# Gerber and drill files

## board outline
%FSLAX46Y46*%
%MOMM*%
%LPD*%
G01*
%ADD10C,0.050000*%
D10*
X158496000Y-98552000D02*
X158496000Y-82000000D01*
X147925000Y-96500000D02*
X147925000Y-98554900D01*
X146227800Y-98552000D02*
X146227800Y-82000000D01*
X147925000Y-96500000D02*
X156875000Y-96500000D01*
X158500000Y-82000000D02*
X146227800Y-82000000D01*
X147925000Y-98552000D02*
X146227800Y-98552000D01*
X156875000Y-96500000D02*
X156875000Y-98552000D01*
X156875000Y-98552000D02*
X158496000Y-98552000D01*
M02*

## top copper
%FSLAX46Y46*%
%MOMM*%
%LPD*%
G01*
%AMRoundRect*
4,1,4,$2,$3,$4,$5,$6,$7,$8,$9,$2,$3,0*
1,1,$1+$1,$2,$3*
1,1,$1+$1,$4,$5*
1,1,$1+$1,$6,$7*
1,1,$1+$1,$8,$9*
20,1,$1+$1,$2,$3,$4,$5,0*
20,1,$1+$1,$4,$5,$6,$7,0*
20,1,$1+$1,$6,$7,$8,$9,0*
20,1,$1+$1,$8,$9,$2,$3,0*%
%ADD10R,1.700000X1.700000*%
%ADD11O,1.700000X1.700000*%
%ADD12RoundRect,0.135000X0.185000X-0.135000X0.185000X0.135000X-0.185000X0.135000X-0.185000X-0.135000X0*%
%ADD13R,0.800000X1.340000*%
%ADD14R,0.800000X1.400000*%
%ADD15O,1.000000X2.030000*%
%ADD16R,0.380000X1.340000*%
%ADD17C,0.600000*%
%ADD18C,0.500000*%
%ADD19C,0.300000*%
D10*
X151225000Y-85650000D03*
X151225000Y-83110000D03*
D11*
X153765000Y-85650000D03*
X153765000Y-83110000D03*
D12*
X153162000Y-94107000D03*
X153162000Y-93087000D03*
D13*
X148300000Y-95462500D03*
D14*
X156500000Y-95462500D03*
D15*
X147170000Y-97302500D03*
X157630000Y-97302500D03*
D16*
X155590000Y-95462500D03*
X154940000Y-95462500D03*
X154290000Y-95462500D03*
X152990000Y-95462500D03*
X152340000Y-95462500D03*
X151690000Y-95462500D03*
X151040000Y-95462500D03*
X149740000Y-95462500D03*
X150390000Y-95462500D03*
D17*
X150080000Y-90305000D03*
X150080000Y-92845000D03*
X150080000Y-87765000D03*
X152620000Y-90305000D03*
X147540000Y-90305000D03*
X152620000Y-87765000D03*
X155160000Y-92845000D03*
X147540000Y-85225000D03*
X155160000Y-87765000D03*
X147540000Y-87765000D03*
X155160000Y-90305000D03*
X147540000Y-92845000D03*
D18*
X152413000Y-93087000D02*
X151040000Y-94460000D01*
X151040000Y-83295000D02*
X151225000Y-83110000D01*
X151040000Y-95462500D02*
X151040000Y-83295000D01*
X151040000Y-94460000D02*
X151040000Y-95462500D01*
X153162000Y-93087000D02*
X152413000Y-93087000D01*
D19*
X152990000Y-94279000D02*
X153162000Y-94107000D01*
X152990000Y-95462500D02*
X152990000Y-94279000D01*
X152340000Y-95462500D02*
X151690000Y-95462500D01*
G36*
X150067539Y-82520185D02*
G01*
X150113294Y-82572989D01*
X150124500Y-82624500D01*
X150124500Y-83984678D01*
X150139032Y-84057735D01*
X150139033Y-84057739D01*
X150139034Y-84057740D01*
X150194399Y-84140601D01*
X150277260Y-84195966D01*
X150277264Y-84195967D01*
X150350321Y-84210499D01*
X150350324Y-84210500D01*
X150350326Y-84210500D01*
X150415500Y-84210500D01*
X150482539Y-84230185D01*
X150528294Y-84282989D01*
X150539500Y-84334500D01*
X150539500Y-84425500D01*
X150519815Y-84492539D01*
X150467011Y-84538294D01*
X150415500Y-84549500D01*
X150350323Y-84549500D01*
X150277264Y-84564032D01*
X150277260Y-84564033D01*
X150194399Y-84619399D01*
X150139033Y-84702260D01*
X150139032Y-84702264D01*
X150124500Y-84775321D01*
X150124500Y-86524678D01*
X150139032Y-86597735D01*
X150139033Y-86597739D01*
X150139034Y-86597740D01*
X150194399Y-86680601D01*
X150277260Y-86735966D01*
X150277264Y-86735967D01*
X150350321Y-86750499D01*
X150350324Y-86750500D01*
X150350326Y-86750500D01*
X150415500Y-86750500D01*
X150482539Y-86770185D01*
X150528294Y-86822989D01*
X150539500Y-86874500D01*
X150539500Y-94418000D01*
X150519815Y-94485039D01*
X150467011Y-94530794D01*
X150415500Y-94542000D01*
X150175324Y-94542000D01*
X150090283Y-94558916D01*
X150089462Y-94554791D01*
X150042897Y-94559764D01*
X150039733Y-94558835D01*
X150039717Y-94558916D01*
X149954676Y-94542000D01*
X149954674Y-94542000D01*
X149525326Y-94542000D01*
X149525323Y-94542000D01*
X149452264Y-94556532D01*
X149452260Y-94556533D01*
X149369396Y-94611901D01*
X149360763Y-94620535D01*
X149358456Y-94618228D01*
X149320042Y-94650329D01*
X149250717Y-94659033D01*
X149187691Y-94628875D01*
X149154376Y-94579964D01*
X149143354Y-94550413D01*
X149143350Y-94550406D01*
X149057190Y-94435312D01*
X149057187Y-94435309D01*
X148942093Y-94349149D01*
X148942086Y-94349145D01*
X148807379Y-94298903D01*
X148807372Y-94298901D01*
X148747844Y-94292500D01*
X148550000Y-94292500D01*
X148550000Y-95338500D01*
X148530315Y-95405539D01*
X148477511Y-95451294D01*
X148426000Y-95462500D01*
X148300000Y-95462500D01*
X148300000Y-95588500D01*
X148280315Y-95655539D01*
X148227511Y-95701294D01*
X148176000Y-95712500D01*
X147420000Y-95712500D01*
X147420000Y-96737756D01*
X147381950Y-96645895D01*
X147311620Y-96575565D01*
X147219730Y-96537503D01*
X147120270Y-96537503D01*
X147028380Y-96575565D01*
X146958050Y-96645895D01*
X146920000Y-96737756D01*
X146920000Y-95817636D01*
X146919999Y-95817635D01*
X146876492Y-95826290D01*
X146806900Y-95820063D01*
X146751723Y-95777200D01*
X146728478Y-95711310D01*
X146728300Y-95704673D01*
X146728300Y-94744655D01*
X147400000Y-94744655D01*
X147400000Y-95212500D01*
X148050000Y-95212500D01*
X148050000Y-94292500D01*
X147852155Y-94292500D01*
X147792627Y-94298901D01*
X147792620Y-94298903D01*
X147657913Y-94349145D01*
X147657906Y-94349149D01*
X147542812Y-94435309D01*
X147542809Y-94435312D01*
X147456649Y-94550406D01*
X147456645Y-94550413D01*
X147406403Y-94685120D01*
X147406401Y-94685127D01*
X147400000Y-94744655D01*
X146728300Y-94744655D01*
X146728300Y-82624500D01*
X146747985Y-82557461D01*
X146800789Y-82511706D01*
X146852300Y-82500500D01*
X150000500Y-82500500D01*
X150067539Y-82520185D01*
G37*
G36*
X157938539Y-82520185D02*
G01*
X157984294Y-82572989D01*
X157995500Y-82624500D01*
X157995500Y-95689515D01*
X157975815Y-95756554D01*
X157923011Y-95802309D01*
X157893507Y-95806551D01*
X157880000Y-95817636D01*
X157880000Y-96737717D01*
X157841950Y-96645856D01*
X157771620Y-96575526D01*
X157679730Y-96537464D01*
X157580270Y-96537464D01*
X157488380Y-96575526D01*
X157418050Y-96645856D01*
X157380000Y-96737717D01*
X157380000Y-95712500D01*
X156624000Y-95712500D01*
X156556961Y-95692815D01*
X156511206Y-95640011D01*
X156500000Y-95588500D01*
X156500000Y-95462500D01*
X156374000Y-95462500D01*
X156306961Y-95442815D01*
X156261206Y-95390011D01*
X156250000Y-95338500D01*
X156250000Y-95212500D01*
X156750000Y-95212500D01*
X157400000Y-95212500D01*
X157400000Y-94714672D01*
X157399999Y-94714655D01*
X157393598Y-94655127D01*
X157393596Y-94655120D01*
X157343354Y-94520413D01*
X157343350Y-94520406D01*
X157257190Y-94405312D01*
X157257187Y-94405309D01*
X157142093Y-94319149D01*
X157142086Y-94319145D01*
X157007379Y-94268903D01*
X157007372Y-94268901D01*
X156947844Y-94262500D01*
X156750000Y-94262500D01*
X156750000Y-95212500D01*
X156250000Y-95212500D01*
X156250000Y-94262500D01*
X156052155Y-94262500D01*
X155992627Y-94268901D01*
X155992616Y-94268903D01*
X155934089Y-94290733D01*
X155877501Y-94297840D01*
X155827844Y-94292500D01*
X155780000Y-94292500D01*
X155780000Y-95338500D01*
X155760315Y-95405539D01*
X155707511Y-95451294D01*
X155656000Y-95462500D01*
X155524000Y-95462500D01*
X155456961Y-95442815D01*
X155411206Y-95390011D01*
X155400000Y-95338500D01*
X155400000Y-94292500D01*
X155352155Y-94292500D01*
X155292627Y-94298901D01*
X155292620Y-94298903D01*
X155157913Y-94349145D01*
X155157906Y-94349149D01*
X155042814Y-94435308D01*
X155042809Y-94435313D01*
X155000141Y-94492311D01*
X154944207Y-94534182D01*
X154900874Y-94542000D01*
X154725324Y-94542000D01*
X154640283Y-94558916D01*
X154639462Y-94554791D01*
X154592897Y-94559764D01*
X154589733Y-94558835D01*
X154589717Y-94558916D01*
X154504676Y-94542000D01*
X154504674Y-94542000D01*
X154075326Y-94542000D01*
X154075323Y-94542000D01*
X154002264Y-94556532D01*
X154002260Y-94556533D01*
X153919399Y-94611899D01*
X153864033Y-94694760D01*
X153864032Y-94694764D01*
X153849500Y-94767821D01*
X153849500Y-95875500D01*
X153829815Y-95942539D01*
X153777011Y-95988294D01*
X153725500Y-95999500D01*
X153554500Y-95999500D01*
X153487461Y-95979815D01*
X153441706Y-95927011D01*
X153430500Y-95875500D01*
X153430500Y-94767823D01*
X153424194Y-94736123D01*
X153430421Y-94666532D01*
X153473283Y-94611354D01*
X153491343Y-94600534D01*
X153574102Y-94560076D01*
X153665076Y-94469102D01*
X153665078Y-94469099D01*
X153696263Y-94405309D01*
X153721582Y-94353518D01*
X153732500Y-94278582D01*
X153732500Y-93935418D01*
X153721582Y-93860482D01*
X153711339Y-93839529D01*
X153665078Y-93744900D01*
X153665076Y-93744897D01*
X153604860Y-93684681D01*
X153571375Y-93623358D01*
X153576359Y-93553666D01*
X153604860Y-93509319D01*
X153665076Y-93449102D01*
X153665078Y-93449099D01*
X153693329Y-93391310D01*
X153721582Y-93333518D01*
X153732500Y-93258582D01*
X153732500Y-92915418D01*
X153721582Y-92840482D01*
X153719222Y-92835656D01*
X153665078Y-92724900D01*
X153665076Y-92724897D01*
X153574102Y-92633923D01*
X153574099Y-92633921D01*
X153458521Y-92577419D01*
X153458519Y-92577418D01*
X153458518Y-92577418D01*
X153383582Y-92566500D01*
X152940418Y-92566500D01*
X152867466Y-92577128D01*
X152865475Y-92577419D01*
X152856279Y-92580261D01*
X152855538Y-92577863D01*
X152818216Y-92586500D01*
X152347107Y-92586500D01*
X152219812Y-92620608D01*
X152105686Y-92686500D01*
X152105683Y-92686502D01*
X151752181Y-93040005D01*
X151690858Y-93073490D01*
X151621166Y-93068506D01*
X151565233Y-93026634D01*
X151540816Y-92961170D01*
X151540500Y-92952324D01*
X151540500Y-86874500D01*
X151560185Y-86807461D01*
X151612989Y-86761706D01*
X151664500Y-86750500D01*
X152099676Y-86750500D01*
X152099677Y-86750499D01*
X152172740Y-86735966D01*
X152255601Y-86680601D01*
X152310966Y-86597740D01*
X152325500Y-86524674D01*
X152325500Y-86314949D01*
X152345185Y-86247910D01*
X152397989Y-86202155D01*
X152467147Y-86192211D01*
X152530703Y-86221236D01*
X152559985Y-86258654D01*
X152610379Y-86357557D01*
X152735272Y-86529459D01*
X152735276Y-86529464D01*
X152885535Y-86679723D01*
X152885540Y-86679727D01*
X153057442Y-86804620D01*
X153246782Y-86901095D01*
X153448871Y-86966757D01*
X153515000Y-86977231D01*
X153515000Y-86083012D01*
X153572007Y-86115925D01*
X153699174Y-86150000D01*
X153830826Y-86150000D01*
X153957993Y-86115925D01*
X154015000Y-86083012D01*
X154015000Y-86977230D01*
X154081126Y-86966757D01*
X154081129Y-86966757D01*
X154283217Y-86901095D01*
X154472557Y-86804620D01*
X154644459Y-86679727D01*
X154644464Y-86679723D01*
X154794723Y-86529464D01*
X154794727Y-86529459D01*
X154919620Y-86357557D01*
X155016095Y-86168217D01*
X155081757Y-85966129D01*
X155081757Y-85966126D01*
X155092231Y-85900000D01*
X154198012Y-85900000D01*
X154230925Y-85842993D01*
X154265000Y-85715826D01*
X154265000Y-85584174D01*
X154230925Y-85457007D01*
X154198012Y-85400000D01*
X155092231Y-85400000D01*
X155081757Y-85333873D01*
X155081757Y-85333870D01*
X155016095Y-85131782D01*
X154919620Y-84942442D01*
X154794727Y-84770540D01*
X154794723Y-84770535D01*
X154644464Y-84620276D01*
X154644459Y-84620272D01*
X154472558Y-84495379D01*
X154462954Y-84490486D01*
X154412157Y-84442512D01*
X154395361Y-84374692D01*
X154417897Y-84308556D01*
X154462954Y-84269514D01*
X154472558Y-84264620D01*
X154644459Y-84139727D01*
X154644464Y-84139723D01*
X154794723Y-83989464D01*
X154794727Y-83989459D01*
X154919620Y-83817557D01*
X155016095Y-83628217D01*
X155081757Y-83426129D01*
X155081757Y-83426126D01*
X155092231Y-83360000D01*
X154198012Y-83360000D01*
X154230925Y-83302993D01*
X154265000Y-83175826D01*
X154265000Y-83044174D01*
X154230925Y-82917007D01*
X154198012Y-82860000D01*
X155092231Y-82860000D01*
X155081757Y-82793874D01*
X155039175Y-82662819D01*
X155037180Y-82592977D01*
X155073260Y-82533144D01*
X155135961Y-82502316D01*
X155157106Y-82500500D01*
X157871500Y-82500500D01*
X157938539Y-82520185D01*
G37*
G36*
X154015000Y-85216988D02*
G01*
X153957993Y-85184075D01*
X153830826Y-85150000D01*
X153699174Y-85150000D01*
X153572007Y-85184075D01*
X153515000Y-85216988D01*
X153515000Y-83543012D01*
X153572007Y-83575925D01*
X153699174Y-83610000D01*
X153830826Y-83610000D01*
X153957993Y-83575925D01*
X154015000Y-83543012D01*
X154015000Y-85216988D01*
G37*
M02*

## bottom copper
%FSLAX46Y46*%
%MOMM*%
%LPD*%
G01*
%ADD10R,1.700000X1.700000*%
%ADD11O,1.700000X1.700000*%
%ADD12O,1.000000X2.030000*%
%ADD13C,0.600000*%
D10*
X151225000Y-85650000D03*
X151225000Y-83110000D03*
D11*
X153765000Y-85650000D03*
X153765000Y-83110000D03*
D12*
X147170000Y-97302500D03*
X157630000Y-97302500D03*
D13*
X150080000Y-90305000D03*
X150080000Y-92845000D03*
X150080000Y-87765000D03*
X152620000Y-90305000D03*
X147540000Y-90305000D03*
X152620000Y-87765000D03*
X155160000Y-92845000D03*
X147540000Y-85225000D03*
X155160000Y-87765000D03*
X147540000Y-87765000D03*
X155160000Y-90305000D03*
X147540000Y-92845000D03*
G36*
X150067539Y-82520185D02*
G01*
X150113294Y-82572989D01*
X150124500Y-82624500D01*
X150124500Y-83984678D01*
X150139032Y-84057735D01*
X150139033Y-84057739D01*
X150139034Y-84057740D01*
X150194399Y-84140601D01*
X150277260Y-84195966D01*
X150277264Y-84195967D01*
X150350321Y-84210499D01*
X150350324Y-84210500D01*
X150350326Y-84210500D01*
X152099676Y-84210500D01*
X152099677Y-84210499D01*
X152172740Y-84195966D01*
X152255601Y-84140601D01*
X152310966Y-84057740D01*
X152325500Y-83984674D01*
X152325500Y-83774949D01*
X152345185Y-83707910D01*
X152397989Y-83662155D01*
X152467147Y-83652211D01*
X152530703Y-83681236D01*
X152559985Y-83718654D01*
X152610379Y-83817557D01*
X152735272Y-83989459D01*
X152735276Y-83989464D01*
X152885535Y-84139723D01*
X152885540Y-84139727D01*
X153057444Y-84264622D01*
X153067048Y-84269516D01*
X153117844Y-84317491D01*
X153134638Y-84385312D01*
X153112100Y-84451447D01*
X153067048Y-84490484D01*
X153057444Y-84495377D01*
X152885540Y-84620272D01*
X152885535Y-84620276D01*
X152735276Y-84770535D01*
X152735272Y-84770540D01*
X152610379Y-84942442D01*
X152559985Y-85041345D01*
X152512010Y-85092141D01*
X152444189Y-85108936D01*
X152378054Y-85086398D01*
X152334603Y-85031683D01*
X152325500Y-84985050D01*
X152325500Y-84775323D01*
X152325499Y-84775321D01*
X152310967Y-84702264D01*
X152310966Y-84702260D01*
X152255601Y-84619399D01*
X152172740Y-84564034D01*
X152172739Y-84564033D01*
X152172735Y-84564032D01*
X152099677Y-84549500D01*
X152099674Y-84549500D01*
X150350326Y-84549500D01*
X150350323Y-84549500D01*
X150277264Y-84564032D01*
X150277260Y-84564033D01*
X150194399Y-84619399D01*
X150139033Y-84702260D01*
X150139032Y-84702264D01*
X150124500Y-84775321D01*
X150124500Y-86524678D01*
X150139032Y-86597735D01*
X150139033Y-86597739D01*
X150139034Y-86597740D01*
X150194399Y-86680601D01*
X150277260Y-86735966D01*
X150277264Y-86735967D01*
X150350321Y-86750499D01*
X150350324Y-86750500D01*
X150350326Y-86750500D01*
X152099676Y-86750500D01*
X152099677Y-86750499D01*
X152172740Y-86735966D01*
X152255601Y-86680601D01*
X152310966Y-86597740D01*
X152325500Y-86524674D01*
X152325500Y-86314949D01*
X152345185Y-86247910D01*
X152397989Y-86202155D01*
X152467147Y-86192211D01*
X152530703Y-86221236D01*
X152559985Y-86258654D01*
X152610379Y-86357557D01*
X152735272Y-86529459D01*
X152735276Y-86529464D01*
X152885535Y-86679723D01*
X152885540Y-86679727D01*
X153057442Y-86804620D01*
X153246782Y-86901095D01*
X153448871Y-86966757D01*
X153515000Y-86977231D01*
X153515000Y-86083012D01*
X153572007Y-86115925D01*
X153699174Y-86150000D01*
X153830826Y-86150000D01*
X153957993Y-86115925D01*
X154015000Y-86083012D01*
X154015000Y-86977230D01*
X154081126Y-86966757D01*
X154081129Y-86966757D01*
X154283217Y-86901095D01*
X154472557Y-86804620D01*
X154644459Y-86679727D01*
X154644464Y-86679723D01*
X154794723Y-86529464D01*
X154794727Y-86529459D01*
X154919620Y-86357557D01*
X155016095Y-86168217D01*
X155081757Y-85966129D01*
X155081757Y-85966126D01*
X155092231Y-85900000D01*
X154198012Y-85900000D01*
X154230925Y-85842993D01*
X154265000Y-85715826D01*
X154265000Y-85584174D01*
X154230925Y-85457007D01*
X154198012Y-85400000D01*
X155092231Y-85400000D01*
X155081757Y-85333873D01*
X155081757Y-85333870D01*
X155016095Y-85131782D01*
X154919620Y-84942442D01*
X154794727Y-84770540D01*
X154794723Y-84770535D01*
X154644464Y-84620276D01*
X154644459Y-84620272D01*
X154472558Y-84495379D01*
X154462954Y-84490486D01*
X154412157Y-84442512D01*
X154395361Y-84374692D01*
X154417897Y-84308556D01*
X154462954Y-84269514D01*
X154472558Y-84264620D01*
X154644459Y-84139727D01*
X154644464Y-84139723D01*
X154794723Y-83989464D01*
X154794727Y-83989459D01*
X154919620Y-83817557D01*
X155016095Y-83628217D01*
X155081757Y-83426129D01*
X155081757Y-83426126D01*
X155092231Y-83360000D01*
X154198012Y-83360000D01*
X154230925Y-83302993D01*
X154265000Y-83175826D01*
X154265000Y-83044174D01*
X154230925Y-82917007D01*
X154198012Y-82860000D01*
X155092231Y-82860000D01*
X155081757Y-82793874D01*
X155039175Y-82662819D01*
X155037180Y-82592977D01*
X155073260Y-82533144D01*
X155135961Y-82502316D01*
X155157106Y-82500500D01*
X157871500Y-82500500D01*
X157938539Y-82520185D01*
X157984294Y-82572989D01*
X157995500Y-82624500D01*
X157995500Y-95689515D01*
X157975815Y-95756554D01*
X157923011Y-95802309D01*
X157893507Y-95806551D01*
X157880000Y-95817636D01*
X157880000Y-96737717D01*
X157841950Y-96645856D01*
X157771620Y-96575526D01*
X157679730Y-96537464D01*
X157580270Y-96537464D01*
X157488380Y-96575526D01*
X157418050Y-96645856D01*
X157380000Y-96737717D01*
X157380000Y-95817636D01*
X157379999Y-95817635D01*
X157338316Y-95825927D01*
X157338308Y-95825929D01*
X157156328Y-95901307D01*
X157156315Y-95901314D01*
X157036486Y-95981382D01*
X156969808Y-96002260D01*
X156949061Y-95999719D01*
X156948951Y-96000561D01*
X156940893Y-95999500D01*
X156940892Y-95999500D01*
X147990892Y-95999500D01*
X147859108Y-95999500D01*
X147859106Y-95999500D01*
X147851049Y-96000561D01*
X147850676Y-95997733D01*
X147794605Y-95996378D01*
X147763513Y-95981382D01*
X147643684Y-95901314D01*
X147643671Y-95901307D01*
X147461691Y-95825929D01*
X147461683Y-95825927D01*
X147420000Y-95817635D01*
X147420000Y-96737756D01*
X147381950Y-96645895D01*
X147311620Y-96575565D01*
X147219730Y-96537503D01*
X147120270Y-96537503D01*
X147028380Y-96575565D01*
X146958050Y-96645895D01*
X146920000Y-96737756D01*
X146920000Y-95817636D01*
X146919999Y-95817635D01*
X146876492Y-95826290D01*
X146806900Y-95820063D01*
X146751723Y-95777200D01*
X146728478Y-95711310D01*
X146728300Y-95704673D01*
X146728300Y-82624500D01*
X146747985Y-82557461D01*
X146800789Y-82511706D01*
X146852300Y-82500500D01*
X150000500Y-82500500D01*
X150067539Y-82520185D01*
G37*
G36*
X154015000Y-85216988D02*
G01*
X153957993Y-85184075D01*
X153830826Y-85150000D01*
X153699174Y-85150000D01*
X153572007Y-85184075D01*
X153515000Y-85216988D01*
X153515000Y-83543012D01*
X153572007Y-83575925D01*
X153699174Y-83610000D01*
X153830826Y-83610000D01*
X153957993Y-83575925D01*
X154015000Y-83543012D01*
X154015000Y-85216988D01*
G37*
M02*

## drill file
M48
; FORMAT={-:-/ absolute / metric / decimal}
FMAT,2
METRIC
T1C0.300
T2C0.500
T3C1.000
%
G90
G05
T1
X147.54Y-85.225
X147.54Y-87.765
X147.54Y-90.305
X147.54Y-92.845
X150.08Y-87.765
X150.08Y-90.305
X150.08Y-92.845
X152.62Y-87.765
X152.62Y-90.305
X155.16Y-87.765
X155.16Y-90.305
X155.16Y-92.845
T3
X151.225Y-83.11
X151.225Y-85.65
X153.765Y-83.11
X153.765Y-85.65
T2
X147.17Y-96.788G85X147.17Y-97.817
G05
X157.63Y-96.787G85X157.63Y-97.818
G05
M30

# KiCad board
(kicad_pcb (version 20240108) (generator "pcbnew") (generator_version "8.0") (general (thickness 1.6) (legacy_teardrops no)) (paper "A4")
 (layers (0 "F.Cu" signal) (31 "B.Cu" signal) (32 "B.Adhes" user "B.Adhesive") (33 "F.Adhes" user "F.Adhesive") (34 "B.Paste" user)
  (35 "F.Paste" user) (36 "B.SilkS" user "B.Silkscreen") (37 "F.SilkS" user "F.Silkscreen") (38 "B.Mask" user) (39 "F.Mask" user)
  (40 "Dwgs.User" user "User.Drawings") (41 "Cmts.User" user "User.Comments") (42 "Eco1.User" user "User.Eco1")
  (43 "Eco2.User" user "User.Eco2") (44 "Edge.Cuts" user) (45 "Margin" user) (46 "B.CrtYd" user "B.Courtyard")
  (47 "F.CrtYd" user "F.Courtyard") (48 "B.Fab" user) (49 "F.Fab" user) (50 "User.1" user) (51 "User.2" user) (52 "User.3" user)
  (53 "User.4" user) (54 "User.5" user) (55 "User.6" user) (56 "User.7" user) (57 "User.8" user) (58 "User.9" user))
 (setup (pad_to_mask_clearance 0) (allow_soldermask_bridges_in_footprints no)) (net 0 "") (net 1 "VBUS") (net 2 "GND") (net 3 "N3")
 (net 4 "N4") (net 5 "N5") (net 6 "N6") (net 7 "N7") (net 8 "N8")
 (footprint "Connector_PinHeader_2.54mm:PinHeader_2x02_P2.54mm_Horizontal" (layer "F.Cu") (at 151.225 85.65 90)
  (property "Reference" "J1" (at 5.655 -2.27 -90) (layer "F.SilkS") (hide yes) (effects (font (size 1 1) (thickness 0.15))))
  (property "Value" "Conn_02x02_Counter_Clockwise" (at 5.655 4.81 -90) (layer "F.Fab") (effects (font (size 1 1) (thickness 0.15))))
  (pad "1" thru_hole rect (at 0 0 90) (size 1.7 1.7) (drill 1) (layers "*.Cu" "*.Mask") (remove_unused_layers no) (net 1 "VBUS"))
  (pad "2" thru_hole rect (at 2.54 0 90) (size 1.7 1.7) (drill 1) (layers "*.Cu" "*.Mask") (remove_unused_layers no) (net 1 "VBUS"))
  (pad "3" thru_hole oval (at 0 2.54 90) (size 1.7 1.7) (drill 1) (layers "*.Cu" "*.Mask") (remove_unused_layers no) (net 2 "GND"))
  (pad "4" thru_hole oval (at 2.54 2.54 90) (size 1.7 1.7) (drill 1) (layers "*.Cu" "*.Mask") (remove_unused_layers no) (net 2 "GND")))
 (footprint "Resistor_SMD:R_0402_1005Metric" (layer "F.Cu") (at 153.162 93.597 90)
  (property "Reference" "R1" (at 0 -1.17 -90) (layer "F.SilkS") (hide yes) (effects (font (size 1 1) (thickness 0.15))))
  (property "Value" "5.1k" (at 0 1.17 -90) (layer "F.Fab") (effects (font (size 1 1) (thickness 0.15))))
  (pad "1" smd roundrect (at -0.51 0 90) (size 0.54 0.64) (layers "F.Cu" "F.Paste" "F.Mask") (roundrect_rratio 0.25) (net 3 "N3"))
  (pad "2" smd roundrect (at 0.51 0 90) (size 0.54 0.64) (layers "F.Cu" "F.Paste" "F.Mask") (roundrect_rratio 0.25) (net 1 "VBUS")))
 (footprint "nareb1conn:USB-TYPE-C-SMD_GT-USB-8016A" (layer "F.Cu") (at 152.4 96.3825)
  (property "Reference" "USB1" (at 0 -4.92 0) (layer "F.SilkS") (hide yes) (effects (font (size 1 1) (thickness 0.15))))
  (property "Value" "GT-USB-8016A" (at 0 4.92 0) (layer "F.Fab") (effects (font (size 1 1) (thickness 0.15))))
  (pad "1" smd rect (at -4.1 -0.92) (size 0.8 1.34) (layers "F.Cu" "F.Paste" "F.Mask") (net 2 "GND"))
  (pad "2" smd rect (at 4.1 -0.92) (size 0.8 1.4) (layers "F.Cu" "F.Paste" "F.Mask") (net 2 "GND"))
  (pad "3" thru_hole oval (at -5.23 0.92) (size 1 2.03) (drill oval 0.500024 1.529994) (layers "*.Cu" "*.Mask") (remove_unused_layers no)
   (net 2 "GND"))
  (pad "4" thru_hole oval (at 5.23 0.92) (size 1 2.03) (drill oval 0.500024 1.530071) (layers "*.Cu" "*.Mask") (remove_unused_layers no)
   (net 2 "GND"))
  (pad "A1" smd rect (at 3.19 -0.92) (size 0.38 1.34) (layers "F.Cu" "F.Paste" "F.Mask") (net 2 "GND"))
  (pad "A2" smd rect (at 2.54 -0.92) (size 0.38 1.34) (layers "F.Cu" "F.Paste" "F.Mask") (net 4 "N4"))
  (pad "A3" smd rect (at 1.89 -0.92) (size 0.38 1.34) (layers "F.Cu" "F.Paste" "F.Mask") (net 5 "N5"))
  (pad "A5" smd rect (at 0.59 -0.92) (size 0.38 1.34) (layers "F.Cu" "F.Paste" "F.Mask") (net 3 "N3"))
  (pad "A6" smd rect (at -0.06 -0.92) (size 0.38 1.34) (layers "F.Cu" "F.Paste" "F.Mask") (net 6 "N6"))
  (pad "A7" smd rect (at -0.71 -0.92) (size 0.38 1.34) (layers "F.Cu" "F.Paste" "F.Mask") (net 6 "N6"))
  (pad "A9" smd rect (at -1.36 -0.92) (size 0.38 1.34) (layers "F.Cu" "F.Paste" "F.Mask") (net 1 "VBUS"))
  (pad "B10" smd rect (at -2.66 -0.92) (size 0.38 1.34) (layers "F.Cu" "F.Paste" "F.Mask") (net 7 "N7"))
  (pad "B11" smd rect (at -2.01 -0.92) (size 0.38 1.34) (layers "F.Cu" "F.Paste" "F.Mask") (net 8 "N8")))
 (gr_line (start 158.496 98.552) (end 158.496 82) (stroke (width 0.05) (type default)) (layer "Edge.Cuts"))
 (gr_line (start 147.925 96.5) (end 147.925 98.5549) (stroke (width 0.05) (type default)) (layer "Edge.Cuts"))
 (gr_line (start 146.2278 98.552) (end 146.2278 82) (stroke (width 0.05) (type default)) (layer "Edge.Cuts"))
 (gr_line (start 147.925 96.5) (end 156.875 96.5) (stroke (width 0.05) (type default)) (layer "Edge.Cuts"))
 (gr_line (start 158.5 82) (end 146.2278 82) (stroke (width 0.05) (type default)) (layer "Edge.Cuts"))
 (gr_line (start 147.925 98.552) (end 146.2278 98.552) (stroke (width 0.05) (type default)) (layer "Edge.Cuts"))
 (gr_line (start 156.875 96.5) (end 156.875 98.552) (stroke (width 0.05) (type default)) (layer "Edge.Cuts"))
 (gr_line (start 156.875 98.552) (end 158.496 98.552) (stroke (width 0.05) (type default)) (layer "Edge.Cuts"))
 (via (at 150.08 90.305) (size 0.6) (drill 0.3) (layers "F.Cu" "B.Cu") (free yes) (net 2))
 (via (at 150.08 92.845) (size 0.6) (drill 0.3) (layers "F.Cu" "B.Cu") (free yes) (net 2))
 (via (at 150.08 87.765) (size 0.6) (drill 0.3) (layers "F.Cu" "B.Cu") (free yes) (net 2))
 (via (at 152.62 90.305) (size 0.6) (drill 0.3) (layers "F.Cu" "B.Cu") (free yes) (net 2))
 (via (at 147.54 90.305) (size 0.6) (drill 0.3) (layers "F.Cu" "B.Cu") (free yes) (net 2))
 (via (at 152.62 87.765) (size 0.6) (drill 0.3) (layers "F.Cu" "B.Cu") (free yes) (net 2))
 (via (at 155.16 92.845) (size 0.6) (drill 0.3) (layers "F.Cu" "B.Cu") (free yes) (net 2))
 (via (at 147.54 85.225) (size 0.6) (drill 0.3) (layers "F.Cu" "B.Cu") (free yes) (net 2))
 (via (at 155.16 87.765) (size 0.6) (drill 0.3) (layers "F.Cu" "B.Cu") (free yes) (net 2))
 (via (at 147.54 87.765) (size 0.6) (drill 0.3) (layers "F.Cu" "B.Cu") (free yes) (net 2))
 (via (at 155.16 90.305) (size 0.6) (drill 0.3) (layers "F.Cu" "B.Cu") (free yes) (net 2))
 (via (at 147.54 92.845) (size 0.6) (drill 0.3) (layers "F.Cu" "B.Cu") (free yes) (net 2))
 (segment (start 152.413 93.087) (end 151.04 94.46) (width 0.5) (layer "F.Cu") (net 1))
 (segment (start 151.04 83.295) (end 151.225 83.11) (width 0.5) (layer "F.Cu") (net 1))
 (segment (start 151.04 95.4625) (end 151.04 83.295) (width 0.5) (layer "F.Cu") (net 1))
 (segment (start 151.04 94.46) (end 151.04 95.4625) (width 0.5) (layer "F.Cu") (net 1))
 (segment (start 153.162 93.087) (end 152.413 93.087) (width 0.5) (layer "F.Cu") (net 1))
 (segment (start 152.99 94.279) (end 153.162 94.107) (width 0.3) (layer "F.Cu") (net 3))
 (segment (start 152.99 95.4625) (end 152.99 94.279) (width 0.3) (layer "F.Cu") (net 3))
 (segment (start 152.34 95.4625) (end 151.69 95.4625) (width 0.3) (layer "F.Cu") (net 6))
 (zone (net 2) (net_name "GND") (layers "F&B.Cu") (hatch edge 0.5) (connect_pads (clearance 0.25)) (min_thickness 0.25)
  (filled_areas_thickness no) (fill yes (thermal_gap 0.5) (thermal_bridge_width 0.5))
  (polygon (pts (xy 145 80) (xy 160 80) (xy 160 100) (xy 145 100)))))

